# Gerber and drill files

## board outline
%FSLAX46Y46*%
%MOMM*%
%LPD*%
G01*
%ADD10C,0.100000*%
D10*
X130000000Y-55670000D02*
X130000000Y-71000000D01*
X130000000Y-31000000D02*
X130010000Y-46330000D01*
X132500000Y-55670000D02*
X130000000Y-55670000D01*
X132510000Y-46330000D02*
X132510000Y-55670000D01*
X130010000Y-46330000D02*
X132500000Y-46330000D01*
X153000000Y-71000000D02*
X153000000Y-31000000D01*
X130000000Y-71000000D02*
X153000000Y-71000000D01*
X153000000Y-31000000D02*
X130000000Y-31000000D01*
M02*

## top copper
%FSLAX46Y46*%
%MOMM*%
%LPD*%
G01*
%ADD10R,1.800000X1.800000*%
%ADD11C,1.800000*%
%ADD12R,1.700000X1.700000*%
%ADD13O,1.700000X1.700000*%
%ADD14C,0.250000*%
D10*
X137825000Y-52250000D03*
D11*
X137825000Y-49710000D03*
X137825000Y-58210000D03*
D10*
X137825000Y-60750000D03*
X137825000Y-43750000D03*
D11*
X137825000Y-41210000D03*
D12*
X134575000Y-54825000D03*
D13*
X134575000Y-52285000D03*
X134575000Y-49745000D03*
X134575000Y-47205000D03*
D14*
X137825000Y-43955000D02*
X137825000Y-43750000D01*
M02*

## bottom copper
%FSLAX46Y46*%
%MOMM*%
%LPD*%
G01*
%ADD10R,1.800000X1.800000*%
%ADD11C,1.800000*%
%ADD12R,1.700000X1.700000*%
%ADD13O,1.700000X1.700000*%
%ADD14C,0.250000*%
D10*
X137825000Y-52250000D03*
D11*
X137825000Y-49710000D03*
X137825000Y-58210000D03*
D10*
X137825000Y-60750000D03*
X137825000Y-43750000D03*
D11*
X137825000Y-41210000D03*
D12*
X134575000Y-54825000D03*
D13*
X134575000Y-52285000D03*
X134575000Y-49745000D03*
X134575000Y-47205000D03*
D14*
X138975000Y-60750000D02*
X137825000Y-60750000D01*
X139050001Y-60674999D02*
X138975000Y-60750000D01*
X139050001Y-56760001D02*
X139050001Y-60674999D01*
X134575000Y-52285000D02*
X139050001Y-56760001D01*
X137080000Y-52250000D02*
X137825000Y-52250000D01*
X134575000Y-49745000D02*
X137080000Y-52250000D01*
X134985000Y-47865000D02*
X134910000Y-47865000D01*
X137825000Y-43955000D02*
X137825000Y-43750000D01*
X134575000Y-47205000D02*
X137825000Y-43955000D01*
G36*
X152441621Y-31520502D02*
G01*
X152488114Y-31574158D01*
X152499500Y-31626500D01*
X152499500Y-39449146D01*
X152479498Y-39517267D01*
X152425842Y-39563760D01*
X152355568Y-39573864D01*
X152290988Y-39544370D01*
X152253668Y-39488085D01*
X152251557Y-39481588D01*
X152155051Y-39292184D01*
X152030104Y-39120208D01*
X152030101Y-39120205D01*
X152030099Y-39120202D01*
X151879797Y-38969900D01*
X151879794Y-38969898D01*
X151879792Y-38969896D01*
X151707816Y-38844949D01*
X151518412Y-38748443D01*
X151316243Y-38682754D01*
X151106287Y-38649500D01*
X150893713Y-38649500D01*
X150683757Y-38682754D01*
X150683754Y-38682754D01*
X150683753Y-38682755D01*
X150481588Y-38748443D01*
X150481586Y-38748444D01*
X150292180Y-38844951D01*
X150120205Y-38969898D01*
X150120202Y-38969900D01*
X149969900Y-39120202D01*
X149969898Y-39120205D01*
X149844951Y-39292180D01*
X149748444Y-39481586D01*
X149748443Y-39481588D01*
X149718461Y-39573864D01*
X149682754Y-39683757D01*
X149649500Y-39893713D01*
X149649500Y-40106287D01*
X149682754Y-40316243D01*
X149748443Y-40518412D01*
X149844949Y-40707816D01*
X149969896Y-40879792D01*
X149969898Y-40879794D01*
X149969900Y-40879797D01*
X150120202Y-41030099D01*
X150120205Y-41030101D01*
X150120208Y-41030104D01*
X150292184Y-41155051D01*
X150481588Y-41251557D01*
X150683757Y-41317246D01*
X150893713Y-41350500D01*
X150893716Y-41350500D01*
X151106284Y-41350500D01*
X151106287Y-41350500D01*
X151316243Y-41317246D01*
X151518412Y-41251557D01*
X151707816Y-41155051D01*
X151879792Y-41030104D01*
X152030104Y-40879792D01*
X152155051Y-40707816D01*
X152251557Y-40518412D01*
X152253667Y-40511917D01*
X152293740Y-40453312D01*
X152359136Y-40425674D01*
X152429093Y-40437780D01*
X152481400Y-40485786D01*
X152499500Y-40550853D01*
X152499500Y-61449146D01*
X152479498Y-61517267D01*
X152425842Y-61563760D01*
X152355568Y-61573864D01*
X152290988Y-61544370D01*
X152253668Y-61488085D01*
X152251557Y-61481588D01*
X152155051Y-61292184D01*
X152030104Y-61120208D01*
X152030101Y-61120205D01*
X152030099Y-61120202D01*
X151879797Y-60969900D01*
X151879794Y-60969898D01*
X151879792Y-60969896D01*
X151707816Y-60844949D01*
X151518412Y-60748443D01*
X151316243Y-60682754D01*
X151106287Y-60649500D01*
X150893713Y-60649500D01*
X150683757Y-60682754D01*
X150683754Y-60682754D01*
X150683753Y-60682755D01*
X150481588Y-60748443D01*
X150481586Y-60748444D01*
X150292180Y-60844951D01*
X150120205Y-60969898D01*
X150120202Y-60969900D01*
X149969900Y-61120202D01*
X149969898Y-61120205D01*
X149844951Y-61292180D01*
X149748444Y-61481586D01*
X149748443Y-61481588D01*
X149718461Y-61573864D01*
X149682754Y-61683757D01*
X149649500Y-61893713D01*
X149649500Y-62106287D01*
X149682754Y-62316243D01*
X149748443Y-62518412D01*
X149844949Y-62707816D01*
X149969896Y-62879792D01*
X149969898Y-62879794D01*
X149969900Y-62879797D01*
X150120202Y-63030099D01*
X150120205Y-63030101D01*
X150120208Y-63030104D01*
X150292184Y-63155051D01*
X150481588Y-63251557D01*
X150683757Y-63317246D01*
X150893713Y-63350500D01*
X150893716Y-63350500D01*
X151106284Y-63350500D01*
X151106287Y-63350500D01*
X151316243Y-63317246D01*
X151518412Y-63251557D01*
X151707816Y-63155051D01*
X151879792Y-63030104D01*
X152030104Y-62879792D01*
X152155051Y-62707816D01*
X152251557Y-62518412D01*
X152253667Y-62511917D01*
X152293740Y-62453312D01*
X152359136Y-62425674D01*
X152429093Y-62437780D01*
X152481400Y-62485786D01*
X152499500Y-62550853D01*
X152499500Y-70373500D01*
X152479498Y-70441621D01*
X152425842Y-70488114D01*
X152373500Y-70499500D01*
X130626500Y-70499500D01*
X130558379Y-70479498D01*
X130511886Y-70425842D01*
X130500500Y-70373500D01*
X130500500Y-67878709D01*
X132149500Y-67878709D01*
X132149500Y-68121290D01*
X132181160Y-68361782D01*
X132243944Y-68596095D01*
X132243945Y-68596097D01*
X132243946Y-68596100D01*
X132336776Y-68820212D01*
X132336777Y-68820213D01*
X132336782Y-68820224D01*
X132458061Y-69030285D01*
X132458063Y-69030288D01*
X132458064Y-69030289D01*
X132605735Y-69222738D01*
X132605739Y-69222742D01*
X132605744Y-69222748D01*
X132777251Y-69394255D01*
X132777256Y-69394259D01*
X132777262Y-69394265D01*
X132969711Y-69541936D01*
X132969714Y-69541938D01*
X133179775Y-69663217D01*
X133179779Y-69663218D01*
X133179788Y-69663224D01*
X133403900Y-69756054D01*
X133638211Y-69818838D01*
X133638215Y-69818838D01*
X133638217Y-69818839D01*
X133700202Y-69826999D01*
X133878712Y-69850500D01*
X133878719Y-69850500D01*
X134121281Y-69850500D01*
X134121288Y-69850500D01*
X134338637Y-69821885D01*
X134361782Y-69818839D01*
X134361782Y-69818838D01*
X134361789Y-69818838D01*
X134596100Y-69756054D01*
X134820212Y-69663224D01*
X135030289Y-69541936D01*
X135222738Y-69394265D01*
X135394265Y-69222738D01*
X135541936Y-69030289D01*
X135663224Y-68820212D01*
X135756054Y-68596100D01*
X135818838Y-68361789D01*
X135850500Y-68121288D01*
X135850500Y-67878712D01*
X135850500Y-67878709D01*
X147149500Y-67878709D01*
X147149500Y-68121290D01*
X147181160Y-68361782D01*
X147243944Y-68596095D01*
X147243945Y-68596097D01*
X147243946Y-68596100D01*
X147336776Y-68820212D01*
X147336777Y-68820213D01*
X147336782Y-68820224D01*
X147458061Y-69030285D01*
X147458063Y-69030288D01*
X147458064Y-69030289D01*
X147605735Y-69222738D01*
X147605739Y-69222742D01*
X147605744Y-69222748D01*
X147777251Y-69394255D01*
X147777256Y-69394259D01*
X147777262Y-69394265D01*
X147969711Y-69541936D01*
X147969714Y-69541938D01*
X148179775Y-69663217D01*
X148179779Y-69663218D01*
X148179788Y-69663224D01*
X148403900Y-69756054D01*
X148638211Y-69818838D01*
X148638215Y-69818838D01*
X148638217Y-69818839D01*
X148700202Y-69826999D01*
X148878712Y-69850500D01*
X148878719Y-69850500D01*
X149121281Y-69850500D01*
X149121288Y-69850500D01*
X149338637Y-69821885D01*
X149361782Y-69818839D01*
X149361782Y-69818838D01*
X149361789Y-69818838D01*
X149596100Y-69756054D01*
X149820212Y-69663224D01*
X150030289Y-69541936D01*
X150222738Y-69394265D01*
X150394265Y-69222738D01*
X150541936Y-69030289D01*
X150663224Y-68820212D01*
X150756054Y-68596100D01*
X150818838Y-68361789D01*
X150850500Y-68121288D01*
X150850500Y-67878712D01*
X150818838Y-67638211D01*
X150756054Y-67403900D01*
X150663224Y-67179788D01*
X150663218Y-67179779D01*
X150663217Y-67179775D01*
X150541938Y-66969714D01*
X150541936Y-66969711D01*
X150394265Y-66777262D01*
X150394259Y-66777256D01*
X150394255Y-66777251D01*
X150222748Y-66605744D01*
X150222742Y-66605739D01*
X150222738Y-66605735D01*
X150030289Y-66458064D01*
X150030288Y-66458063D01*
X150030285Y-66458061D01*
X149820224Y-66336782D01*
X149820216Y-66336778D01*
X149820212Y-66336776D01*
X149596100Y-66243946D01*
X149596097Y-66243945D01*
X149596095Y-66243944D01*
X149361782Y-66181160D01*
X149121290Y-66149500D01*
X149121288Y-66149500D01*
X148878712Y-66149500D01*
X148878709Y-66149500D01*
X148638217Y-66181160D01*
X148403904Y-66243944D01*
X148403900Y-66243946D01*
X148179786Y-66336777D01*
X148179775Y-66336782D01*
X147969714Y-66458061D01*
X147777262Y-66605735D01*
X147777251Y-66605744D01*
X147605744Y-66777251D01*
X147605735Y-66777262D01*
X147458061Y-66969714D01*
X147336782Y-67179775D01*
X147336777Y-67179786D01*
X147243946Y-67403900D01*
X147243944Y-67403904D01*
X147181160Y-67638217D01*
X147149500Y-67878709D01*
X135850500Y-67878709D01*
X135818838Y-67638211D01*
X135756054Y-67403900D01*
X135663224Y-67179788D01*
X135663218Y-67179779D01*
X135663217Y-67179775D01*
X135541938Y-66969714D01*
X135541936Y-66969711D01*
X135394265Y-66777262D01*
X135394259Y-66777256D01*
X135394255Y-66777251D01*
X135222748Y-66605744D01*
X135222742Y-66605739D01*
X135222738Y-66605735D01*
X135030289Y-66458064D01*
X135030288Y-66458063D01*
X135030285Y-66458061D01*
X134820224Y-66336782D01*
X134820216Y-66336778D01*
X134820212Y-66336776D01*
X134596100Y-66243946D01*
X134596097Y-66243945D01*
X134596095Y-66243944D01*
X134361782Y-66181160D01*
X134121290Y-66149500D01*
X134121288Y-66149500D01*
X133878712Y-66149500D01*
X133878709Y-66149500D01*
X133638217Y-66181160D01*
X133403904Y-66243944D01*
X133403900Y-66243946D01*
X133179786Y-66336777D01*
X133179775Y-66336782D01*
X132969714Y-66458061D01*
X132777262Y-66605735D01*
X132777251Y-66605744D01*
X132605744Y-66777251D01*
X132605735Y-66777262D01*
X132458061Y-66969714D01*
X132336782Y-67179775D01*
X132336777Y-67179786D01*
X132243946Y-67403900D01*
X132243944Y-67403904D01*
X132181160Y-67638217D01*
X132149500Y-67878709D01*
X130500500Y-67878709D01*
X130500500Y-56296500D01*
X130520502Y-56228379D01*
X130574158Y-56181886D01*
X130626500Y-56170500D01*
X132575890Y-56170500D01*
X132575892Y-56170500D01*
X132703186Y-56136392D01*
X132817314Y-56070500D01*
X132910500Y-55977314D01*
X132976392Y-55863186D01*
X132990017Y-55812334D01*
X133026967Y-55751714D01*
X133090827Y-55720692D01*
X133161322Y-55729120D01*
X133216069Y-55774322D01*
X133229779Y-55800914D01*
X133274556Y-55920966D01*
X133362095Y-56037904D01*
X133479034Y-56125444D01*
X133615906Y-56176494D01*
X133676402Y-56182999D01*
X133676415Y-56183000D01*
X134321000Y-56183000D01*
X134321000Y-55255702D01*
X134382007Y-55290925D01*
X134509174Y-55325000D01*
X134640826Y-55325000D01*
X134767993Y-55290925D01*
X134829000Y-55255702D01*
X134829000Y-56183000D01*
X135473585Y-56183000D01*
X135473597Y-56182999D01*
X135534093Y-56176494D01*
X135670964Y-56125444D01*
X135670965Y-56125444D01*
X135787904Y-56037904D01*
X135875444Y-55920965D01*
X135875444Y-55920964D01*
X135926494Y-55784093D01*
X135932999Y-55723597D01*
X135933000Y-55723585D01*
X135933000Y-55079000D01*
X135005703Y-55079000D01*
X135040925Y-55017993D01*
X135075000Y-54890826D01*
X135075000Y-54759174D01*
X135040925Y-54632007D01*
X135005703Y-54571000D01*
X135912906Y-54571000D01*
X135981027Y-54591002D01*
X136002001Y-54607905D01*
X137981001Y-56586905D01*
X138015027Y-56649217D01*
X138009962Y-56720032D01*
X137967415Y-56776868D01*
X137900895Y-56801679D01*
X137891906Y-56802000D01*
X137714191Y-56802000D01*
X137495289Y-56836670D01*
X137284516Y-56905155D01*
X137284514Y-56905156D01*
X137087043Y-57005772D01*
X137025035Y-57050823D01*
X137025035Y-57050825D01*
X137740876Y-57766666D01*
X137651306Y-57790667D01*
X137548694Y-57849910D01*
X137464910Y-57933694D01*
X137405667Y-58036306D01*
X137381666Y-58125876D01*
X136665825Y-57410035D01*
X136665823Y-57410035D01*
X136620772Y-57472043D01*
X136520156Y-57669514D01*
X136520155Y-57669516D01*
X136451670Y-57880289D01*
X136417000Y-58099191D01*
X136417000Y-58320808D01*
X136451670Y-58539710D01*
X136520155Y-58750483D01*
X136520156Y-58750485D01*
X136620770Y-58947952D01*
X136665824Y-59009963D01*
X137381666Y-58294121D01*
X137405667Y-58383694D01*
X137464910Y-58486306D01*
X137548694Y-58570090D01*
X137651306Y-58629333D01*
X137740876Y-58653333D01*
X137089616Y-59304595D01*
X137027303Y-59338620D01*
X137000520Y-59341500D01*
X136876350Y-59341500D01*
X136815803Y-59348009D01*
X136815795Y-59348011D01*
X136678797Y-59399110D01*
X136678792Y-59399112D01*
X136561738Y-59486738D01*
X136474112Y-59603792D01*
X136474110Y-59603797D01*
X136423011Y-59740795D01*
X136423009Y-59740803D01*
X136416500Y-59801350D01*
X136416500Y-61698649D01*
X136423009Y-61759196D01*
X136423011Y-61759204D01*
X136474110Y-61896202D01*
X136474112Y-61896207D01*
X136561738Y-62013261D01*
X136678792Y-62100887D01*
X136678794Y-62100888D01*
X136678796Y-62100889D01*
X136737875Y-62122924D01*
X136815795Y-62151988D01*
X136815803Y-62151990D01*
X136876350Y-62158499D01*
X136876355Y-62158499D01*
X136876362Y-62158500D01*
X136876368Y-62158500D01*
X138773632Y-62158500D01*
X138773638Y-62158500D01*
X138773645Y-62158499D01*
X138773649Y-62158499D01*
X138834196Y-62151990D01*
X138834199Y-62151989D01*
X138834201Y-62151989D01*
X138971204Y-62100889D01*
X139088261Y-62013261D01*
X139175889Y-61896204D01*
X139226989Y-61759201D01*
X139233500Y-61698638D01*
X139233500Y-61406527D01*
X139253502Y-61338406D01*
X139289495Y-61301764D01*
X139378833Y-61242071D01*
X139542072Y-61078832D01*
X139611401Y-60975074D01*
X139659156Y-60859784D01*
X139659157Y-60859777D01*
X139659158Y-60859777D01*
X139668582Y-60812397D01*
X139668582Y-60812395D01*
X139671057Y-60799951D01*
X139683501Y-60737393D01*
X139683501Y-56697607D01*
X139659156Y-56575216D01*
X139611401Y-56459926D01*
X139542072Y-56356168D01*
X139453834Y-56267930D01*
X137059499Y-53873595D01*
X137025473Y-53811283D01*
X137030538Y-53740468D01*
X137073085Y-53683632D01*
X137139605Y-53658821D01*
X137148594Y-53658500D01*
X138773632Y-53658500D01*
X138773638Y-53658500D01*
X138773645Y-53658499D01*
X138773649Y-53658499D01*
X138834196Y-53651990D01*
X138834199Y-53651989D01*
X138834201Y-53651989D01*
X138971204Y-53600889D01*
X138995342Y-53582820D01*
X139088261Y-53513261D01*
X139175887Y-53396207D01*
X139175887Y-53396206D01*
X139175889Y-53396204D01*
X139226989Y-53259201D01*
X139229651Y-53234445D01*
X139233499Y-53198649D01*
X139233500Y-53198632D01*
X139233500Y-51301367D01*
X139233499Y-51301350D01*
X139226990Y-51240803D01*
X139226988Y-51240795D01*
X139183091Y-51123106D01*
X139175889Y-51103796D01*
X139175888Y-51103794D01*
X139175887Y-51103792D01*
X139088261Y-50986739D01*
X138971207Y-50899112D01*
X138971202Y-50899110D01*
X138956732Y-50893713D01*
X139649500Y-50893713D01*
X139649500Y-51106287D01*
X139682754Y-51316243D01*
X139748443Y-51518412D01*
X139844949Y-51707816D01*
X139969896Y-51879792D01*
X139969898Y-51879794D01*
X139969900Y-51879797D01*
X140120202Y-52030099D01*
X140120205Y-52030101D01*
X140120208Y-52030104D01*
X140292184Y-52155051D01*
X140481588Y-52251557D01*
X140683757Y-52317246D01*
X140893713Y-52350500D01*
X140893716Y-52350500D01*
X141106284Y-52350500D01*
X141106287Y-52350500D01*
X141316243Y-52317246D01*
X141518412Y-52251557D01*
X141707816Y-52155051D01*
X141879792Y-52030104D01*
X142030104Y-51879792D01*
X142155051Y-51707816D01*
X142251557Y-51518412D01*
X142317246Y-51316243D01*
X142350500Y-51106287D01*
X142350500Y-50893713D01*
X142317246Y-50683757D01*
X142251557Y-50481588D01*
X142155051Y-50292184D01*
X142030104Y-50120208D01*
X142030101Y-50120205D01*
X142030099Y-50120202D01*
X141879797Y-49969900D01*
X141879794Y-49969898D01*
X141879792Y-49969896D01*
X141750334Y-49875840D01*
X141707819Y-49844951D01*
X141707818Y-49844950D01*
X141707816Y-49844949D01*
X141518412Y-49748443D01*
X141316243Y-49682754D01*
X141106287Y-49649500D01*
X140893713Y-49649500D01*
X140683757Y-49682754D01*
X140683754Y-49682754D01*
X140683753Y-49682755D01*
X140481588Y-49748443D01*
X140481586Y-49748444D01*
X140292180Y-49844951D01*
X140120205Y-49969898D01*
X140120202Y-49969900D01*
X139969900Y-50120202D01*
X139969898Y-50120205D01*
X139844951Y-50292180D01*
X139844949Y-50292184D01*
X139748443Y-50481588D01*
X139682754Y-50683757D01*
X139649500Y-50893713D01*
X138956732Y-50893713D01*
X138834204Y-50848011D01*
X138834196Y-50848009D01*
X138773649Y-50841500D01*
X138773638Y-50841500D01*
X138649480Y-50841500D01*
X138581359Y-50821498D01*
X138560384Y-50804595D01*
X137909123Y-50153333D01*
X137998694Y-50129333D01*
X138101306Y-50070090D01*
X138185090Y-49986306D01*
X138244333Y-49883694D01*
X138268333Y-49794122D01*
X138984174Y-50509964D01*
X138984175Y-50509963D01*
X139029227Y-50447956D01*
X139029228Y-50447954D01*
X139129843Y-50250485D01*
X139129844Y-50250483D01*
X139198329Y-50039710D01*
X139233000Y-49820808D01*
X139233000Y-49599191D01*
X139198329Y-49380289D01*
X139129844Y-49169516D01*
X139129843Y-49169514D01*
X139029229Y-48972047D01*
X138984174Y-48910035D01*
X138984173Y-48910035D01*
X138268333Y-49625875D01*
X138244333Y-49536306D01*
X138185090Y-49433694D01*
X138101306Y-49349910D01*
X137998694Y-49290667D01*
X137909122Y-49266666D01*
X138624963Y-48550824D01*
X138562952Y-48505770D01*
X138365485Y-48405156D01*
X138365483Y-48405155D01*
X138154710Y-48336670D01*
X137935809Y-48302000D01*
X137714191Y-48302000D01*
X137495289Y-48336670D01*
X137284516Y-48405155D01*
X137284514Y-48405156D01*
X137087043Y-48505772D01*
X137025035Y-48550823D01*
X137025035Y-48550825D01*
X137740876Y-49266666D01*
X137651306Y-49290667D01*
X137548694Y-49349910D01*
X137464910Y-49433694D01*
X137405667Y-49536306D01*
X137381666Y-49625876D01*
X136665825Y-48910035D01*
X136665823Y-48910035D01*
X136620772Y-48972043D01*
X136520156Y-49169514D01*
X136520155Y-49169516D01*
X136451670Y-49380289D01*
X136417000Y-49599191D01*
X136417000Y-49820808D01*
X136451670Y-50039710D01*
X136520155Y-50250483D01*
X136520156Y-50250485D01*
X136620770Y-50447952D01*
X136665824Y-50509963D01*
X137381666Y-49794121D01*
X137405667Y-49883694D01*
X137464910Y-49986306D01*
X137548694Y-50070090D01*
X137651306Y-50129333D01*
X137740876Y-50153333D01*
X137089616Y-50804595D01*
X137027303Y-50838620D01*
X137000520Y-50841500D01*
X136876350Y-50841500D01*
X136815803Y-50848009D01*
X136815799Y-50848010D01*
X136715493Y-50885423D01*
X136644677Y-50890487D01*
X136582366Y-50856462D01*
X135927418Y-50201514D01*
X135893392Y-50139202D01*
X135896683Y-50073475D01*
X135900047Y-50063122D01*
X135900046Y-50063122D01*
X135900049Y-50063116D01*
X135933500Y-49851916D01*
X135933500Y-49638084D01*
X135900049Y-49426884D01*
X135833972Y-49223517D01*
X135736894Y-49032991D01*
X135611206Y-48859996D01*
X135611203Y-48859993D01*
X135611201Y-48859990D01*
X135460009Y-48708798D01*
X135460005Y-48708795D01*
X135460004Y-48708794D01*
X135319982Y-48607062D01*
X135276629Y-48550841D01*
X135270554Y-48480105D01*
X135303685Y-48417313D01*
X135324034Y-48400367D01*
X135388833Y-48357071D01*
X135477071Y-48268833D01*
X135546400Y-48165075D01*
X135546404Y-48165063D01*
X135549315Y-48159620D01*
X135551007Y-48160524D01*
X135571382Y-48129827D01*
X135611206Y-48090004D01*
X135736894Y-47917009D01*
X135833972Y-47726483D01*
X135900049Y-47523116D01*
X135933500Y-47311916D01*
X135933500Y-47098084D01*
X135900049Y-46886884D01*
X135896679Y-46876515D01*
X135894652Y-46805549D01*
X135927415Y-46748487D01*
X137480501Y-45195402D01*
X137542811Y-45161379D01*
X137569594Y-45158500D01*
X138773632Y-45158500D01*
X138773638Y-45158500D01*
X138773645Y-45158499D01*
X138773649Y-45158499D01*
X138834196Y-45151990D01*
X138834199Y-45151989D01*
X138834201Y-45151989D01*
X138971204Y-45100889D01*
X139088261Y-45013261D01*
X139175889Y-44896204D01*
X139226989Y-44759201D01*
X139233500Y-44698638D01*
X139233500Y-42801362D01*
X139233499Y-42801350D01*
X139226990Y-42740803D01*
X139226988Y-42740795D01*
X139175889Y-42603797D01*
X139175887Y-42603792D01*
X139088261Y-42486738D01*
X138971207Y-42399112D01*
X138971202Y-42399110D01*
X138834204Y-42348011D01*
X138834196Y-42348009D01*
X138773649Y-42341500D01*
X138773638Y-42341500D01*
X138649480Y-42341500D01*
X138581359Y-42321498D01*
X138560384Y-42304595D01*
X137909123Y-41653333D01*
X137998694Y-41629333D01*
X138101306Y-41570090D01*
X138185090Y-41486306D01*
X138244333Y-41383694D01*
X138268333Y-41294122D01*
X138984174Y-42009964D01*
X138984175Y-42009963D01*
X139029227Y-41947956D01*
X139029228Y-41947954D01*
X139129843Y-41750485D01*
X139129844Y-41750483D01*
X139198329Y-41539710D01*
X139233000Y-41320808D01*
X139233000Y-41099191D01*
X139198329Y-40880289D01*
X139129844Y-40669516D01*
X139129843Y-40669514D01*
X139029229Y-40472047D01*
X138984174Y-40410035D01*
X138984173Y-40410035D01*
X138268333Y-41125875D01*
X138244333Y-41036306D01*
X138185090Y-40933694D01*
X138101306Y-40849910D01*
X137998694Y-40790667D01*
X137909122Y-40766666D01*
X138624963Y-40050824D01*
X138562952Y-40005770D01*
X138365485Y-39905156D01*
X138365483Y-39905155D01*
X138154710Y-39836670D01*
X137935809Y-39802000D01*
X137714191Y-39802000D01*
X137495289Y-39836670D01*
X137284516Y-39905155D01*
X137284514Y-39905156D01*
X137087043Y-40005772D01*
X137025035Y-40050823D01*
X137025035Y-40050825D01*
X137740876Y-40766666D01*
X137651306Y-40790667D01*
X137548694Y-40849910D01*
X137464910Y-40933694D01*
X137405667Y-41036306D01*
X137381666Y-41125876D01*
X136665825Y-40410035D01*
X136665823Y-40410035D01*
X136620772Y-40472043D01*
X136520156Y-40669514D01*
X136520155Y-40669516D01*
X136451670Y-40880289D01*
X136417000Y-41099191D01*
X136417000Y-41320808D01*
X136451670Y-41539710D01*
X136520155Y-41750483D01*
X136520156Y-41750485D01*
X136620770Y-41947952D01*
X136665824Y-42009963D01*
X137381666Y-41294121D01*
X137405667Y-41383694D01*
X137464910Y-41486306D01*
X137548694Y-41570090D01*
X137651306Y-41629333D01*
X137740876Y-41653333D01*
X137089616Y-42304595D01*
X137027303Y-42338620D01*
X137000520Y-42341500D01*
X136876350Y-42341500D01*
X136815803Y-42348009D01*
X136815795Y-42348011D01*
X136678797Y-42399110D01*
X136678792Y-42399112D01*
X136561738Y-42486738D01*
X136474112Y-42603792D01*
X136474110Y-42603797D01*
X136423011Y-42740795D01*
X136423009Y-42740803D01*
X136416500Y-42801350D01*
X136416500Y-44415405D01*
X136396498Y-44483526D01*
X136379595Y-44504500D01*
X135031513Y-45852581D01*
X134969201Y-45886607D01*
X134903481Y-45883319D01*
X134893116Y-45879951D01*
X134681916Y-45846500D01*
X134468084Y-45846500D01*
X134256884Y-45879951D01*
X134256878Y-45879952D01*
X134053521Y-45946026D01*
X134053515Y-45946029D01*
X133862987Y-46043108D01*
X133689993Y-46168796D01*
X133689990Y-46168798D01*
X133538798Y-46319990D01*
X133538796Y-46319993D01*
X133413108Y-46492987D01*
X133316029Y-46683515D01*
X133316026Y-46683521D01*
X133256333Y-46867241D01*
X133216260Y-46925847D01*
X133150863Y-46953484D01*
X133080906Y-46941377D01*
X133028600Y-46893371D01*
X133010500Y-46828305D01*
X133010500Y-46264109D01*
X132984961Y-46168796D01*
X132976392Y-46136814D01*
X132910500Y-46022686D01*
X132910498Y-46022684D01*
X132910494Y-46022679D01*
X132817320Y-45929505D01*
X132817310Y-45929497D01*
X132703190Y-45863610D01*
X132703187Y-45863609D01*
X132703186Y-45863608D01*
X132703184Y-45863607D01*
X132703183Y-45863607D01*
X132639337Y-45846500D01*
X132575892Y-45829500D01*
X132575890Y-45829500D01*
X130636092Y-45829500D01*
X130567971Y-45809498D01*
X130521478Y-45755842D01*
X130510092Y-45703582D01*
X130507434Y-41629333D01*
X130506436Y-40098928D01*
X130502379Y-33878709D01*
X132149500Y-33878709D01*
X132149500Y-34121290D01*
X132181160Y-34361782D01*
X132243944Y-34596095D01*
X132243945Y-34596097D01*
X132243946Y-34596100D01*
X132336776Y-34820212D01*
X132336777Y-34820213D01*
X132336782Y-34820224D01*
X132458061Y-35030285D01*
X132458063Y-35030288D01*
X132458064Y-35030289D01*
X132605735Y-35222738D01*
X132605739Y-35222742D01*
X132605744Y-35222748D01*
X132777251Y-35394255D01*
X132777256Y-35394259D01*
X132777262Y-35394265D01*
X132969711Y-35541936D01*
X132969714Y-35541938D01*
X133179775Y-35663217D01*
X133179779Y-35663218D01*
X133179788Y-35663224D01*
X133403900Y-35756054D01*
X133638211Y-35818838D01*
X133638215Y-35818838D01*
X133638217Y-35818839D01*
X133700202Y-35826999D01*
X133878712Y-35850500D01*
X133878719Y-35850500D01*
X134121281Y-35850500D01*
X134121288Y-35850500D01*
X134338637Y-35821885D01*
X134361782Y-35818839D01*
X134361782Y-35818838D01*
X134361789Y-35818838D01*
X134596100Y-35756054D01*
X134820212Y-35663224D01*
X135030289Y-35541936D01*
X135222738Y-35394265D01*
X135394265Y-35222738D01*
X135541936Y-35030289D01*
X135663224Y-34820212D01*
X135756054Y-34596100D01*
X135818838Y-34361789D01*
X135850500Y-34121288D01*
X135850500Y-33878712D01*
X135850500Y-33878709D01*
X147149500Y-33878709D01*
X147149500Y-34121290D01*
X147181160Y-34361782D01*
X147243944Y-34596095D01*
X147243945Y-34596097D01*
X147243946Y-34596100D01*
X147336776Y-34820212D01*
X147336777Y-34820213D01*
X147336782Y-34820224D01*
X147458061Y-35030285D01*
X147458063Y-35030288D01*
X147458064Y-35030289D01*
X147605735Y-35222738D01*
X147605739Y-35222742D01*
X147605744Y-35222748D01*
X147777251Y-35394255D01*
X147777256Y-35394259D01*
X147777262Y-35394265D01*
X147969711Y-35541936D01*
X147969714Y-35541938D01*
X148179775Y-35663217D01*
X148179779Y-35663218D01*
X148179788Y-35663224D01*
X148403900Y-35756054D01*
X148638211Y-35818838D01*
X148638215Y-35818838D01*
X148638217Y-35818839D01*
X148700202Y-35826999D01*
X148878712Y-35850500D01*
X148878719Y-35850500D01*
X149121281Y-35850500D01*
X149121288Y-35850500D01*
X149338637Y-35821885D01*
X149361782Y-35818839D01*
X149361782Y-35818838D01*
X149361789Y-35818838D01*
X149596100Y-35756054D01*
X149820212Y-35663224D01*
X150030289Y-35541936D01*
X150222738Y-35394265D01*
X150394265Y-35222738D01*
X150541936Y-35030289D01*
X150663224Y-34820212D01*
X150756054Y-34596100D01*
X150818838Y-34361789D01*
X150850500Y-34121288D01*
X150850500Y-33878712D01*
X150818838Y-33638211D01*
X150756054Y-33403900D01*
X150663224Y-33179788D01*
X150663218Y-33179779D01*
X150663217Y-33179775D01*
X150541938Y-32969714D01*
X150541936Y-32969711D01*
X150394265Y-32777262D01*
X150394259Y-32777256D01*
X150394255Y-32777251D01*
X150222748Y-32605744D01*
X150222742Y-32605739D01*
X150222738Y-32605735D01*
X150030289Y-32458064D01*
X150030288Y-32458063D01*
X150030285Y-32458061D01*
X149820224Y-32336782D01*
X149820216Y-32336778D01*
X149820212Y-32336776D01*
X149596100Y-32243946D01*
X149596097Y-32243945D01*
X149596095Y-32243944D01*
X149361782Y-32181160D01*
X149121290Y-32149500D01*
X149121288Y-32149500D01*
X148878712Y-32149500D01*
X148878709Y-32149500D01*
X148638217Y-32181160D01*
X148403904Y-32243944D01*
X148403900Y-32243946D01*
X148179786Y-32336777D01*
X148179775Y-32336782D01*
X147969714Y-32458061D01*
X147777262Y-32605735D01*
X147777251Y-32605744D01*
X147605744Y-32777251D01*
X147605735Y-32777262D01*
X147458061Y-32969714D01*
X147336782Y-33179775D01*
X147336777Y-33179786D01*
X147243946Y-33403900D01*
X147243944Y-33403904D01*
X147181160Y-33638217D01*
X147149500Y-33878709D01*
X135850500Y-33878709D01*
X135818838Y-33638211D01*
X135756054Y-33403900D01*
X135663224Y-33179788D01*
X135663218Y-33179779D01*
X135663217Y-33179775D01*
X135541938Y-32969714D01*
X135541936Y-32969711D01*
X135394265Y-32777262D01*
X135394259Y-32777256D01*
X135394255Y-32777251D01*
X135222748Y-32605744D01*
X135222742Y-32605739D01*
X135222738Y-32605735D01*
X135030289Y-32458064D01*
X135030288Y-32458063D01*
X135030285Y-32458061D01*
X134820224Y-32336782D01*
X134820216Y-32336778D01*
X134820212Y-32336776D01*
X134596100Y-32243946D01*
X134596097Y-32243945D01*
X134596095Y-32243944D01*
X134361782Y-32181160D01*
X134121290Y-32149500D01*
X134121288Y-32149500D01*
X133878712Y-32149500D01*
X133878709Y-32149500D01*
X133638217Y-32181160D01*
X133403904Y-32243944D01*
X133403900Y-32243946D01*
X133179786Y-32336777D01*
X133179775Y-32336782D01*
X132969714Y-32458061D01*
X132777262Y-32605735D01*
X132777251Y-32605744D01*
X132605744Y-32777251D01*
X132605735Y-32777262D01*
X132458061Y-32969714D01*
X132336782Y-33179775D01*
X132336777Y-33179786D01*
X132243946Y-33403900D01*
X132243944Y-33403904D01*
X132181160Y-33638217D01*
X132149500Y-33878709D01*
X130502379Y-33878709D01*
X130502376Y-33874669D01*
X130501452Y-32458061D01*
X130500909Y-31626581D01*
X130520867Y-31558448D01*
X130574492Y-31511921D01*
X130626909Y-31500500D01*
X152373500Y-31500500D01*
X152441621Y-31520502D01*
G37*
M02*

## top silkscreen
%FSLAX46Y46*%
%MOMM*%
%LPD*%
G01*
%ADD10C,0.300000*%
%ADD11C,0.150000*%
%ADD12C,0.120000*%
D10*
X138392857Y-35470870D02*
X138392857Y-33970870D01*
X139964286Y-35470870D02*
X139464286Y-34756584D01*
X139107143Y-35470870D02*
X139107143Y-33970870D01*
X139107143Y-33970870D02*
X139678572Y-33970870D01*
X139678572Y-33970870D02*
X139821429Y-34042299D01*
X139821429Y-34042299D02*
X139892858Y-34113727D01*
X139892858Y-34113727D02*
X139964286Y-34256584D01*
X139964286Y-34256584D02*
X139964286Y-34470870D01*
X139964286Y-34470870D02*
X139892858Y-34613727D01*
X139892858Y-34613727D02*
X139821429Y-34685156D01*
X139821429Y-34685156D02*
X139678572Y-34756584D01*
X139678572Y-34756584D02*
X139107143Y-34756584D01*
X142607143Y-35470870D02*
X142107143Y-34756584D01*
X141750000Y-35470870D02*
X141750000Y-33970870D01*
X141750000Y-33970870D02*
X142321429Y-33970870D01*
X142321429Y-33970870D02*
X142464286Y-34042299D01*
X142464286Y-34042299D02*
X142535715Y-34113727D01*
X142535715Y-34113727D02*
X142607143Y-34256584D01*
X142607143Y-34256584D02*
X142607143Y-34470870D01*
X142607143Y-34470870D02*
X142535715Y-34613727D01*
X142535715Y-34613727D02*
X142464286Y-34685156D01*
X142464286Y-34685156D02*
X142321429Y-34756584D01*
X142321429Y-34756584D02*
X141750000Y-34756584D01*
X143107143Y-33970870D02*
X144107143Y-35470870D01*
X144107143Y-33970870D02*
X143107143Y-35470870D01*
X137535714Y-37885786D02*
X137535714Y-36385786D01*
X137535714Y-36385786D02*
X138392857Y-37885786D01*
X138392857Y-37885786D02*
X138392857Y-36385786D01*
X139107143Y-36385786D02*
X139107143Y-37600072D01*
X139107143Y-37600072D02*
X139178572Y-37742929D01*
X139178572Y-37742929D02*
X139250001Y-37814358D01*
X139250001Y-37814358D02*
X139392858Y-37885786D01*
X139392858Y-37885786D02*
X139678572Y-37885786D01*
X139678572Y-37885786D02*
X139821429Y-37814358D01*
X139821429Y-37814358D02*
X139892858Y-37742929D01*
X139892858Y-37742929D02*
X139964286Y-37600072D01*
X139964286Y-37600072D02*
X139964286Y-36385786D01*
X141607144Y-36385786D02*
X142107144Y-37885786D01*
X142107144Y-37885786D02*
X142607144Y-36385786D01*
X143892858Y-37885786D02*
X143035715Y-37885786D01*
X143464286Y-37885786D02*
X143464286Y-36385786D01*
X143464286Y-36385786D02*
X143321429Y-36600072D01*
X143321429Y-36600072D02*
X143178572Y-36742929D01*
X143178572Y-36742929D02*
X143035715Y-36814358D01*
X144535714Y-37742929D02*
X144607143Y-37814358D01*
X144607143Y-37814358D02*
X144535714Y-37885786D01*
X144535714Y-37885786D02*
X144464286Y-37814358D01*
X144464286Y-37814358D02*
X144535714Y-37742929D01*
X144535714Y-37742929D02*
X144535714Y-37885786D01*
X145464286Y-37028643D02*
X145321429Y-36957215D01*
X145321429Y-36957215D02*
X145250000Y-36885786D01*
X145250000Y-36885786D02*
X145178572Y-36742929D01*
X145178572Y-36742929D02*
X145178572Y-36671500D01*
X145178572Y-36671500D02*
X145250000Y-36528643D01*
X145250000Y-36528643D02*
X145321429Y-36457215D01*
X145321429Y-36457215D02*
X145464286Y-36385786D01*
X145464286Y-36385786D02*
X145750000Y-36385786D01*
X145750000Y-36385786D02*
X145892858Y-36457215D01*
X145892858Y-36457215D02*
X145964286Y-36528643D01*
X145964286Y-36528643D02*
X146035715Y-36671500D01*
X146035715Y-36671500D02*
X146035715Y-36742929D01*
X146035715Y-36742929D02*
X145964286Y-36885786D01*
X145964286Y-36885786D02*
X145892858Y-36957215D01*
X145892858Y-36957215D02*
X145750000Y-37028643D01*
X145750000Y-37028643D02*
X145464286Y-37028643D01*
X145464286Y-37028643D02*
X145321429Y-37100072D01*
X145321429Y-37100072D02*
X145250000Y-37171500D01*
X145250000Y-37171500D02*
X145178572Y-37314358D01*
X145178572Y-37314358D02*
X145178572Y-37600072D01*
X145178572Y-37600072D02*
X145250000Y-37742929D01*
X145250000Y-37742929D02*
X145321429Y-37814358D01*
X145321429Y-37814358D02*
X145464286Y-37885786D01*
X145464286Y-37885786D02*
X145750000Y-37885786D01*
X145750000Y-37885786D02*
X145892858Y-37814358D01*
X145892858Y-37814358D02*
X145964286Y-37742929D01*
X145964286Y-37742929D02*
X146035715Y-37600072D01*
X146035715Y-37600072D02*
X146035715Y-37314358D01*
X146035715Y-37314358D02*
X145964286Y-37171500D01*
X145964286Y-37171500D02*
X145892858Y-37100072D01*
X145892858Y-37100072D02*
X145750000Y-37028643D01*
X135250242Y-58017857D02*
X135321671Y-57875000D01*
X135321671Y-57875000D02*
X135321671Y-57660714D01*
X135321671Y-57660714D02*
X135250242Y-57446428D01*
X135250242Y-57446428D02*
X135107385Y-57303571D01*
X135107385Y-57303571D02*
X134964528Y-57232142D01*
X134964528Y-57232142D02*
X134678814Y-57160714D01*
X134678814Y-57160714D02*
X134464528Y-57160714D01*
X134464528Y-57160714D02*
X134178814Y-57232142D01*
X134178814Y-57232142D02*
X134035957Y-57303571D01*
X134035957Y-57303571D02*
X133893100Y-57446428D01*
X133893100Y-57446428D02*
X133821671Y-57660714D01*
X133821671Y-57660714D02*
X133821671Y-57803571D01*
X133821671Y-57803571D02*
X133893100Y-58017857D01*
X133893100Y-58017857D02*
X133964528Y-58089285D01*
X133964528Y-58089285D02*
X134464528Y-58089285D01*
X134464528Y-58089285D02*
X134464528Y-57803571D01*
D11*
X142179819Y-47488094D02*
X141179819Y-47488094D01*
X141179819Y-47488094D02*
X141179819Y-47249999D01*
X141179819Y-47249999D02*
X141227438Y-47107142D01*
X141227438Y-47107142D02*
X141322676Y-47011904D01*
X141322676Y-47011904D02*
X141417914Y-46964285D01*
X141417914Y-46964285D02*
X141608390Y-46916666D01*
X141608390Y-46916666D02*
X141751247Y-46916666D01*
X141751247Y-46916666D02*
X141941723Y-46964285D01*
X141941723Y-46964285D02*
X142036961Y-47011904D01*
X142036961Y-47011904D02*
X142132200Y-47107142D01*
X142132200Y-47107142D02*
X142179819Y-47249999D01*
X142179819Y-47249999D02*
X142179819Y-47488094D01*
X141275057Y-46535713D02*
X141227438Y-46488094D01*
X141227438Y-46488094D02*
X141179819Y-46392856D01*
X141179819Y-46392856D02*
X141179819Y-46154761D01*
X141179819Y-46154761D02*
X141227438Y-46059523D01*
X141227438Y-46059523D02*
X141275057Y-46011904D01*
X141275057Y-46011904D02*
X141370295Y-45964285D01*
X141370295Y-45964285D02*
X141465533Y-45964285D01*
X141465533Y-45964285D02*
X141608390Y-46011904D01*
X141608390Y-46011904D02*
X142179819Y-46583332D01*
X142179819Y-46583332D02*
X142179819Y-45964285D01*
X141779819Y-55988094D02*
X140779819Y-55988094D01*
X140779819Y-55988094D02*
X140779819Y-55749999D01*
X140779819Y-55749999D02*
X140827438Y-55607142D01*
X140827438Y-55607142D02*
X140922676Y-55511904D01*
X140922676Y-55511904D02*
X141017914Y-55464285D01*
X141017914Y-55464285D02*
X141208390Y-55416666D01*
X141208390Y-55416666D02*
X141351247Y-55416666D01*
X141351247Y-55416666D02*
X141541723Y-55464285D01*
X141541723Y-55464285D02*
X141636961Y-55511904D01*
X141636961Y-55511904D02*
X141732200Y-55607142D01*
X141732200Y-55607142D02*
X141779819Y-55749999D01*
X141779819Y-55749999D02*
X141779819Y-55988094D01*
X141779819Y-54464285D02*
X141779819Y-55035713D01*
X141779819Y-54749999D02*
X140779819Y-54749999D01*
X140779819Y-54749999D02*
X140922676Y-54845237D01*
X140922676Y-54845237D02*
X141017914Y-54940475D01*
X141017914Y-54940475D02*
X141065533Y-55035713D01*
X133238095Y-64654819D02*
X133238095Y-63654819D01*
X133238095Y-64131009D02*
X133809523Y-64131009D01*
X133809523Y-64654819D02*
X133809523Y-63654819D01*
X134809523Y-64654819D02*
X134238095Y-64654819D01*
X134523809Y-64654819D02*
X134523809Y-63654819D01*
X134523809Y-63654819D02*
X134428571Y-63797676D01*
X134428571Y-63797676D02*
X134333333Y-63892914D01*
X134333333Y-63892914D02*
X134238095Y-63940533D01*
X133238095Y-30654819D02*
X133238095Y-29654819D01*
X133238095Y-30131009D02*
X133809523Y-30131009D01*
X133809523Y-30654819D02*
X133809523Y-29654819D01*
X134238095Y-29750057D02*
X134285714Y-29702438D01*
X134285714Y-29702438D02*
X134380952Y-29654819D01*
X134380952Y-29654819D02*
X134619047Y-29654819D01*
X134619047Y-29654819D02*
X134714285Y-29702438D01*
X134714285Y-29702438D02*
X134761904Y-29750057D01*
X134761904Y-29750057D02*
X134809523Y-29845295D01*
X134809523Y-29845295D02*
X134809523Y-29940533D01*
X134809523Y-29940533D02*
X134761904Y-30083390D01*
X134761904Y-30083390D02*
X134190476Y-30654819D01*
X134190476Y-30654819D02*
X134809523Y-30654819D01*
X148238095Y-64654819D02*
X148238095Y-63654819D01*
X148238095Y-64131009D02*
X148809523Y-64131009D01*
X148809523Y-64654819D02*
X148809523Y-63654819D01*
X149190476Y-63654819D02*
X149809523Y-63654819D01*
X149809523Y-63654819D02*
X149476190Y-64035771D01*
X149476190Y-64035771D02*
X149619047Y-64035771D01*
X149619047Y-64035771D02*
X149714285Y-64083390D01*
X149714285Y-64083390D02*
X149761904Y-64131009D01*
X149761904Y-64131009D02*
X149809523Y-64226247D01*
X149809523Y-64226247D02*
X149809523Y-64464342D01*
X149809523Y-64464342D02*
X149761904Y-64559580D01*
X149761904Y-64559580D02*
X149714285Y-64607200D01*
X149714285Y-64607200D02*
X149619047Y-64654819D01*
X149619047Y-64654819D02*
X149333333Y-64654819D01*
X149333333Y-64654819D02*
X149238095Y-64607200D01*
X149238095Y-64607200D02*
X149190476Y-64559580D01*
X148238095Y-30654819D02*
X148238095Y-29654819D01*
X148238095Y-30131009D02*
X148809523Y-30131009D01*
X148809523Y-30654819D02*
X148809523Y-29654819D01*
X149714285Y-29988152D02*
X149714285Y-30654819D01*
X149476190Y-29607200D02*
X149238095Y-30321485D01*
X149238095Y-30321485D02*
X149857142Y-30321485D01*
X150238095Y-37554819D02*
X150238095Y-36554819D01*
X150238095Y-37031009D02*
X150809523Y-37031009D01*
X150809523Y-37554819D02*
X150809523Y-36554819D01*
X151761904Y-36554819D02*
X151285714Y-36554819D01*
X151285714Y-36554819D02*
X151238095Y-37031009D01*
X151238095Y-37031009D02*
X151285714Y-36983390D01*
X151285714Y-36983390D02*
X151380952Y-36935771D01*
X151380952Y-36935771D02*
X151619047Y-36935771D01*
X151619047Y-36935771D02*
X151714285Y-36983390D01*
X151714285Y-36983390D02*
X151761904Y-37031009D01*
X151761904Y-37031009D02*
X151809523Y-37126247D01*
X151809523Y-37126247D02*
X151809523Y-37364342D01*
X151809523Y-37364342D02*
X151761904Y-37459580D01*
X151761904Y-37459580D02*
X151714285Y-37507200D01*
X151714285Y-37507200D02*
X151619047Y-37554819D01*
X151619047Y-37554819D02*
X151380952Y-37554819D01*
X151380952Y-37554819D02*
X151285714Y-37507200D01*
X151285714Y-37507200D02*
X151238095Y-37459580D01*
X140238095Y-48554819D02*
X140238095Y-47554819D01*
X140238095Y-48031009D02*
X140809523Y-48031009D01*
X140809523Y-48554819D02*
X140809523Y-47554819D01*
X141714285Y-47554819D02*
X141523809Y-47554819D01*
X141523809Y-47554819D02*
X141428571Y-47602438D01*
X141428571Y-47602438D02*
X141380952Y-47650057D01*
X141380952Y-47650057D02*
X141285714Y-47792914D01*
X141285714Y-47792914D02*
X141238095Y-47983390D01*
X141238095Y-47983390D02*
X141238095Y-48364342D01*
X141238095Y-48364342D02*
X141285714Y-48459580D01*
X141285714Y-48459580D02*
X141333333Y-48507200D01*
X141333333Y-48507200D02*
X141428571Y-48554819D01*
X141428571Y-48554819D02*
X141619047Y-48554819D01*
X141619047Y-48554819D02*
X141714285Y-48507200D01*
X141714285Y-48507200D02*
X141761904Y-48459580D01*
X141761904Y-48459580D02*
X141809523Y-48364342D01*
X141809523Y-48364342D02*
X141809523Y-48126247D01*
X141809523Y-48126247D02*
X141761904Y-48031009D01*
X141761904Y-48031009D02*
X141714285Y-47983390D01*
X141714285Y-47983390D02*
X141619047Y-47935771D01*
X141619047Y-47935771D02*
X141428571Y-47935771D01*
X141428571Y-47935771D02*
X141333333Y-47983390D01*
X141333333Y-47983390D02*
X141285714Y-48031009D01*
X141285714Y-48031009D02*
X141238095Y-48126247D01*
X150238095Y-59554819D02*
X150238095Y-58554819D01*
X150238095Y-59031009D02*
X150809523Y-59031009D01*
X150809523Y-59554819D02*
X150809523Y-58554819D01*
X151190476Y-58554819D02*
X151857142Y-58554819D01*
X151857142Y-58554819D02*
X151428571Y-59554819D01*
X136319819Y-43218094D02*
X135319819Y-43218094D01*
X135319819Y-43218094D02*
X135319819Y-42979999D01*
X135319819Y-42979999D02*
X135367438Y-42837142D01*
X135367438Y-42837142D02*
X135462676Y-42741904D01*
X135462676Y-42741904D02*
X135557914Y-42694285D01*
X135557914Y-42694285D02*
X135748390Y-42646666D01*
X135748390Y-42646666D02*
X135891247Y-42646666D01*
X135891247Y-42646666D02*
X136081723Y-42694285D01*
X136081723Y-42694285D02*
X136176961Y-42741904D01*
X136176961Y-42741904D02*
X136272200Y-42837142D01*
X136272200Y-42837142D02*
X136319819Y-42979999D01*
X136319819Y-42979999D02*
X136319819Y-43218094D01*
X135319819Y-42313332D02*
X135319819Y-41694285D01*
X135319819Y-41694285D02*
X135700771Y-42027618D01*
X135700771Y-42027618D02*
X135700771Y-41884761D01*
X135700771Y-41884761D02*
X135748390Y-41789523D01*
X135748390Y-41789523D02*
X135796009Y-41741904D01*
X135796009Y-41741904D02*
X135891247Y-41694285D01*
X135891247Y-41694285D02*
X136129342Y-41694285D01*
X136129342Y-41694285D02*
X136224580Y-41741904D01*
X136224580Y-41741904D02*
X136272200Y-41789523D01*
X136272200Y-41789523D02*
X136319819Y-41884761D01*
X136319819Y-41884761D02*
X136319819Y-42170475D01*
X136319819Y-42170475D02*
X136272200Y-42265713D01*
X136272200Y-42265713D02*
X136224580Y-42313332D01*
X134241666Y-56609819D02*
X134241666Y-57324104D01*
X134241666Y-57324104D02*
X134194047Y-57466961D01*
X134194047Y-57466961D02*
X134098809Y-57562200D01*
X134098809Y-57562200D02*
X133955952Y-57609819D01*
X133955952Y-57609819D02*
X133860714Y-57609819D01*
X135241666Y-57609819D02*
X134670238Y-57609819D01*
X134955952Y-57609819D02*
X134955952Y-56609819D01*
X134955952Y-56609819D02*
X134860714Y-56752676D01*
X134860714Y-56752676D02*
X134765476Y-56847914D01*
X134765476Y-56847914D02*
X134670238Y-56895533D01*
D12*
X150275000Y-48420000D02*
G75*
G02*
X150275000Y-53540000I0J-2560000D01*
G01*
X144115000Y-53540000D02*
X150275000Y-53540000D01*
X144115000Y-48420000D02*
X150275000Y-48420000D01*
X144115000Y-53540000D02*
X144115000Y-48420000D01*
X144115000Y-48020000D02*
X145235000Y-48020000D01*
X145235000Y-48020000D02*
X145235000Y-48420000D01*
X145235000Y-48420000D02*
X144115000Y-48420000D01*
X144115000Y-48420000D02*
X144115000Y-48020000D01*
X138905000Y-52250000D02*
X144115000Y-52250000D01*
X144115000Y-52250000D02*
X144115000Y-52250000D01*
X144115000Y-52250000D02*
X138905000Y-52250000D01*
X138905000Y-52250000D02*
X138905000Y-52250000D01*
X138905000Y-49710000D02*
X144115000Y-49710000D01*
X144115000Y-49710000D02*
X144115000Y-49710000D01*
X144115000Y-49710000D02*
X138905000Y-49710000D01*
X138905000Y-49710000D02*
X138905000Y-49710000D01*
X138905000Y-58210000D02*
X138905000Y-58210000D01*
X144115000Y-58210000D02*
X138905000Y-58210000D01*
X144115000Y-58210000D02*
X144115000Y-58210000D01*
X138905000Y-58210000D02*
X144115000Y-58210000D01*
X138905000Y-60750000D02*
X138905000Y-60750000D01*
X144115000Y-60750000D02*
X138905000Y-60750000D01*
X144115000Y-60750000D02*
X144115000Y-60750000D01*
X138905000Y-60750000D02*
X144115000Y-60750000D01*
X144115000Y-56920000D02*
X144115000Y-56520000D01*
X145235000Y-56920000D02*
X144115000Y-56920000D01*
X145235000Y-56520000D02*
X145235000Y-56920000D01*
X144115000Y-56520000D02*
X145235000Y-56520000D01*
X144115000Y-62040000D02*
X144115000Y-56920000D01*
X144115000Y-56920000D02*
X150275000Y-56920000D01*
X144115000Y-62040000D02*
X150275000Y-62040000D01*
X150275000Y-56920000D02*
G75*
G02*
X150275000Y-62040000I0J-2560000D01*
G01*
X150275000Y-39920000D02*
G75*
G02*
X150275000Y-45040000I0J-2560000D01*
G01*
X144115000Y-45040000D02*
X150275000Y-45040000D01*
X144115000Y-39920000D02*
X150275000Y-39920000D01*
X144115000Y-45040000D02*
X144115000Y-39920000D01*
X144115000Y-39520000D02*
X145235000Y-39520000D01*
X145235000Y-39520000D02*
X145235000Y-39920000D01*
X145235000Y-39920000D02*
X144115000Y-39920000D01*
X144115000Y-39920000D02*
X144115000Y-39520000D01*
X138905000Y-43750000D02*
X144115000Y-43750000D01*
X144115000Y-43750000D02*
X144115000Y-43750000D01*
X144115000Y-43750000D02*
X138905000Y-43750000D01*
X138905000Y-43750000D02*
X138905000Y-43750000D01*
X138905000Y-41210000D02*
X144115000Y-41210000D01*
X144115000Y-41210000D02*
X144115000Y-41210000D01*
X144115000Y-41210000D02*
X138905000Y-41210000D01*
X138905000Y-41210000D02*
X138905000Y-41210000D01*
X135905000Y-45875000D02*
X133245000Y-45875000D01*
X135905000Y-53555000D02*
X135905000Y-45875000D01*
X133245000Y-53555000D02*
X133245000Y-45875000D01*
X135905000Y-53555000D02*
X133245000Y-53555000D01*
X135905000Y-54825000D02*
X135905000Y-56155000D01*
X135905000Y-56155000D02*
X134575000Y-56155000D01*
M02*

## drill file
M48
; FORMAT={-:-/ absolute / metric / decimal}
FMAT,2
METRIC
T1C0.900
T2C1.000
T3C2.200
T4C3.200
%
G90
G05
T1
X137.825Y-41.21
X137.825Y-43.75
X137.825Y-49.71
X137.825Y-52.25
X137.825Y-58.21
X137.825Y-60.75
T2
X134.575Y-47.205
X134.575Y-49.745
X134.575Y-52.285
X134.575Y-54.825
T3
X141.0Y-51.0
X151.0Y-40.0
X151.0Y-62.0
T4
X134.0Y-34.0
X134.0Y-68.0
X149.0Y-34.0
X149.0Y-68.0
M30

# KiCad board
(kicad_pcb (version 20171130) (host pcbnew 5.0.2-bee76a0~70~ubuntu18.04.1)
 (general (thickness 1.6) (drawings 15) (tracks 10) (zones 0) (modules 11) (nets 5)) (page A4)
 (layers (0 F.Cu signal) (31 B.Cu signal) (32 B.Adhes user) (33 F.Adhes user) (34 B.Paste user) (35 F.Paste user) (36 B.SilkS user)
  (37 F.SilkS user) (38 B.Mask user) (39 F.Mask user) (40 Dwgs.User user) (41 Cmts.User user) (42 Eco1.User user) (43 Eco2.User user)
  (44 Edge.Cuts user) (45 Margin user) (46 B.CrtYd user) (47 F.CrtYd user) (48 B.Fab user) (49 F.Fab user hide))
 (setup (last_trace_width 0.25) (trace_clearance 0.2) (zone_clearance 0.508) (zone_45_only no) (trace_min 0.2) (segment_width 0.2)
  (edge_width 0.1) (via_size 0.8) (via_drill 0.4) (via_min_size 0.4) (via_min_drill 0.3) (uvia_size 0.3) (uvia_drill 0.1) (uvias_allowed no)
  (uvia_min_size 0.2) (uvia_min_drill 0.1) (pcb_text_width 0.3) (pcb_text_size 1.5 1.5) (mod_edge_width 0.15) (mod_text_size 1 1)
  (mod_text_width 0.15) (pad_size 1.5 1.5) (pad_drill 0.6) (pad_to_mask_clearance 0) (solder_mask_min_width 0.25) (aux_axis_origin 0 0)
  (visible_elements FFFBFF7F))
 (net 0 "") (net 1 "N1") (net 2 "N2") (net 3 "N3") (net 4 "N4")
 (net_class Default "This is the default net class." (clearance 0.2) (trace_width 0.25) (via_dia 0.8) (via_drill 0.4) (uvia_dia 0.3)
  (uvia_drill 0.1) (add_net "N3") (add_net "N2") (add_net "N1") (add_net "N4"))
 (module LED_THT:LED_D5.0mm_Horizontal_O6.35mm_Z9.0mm (layer F.Cu) (at 137.825 52.25 90)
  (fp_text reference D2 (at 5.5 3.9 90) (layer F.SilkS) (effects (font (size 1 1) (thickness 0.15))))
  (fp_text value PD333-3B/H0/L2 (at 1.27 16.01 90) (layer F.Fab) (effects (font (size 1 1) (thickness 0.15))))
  (fp_arc (start 1.27 12.45) (end -1.29 12.45) (angle -180) (layer F.SilkS) (width 0.12))
  (fp_line (start -1.29 6.29) (end -1.29 12.45) (layer F.SilkS) (width 0.12))
  (fp_line (start 3.83 6.29) (end 3.83 12.45) (layer F.SilkS) (width 0.12))
  (fp_line (start -1.29 6.29) (end 3.83 6.29) (layer F.SilkS) (width 0.12))
  (fp_line (start 4.23 6.29) (end 4.23 7.41) (layer F.SilkS) (width 0.12))
  (fp_line (start 4.23 7.41) (end 3.83 7.41) (layer F.SilkS) (width 0.12))
  (fp_line (start 3.83 7.41) (end 3.83 6.29) (layer F.SilkS) (width 0.12))
  (fp_line (start 3.83 6.29) (end 4.23 6.29) (layer F.SilkS) (width 0.12))
  (fp_line (start 0 1.08) (end 0 6.29) (layer F.SilkS) (width 0.12))
  (fp_line (start 0 6.29) (end 0 6.29) (layer F.SilkS) (width 0.12))
  (fp_line (start 0 6.29) (end 0 1.08) (layer F.SilkS) (width 0.12))
  (fp_line (start 0 1.08) (end 0 1.08) (layer F.SilkS) (width 0.12))
  (fp_line (start 2.54 1.08) (end 2.54 6.29) (layer F.SilkS) (width 0.12))
  (fp_line (start 2.54 6.29) (end 2.54 6.29) (layer F.SilkS) (width 0.12))
  (fp_line (start 2.54 6.29) (end 2.54 1.08) (layer F.SilkS) (width 0.12))
  (fp_line (start 2.54 1.08) (end 2.54 1.08) (layer F.SilkS) (width 0.12))
  (pad 1 thru_hole rect (at 0 0 90) (size 1.8 1.8) (drill 0.9) (layers *.Cu *.Mask) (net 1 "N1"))
  (pad 2 thru_hole circle (at 2.54 0 90) (size 1.8 1.8) (drill 0.9) (layers *.Cu *.Mask) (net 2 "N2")))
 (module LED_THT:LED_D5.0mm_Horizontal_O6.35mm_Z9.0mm (layer F.Cu) (at 137.825 60.75 90)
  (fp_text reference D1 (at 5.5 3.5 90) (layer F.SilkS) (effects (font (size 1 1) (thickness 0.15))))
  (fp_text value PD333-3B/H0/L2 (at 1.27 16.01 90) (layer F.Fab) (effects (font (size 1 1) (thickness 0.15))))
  (fp_line (start 2.54 1.08) (end 2.54 1.08) (layer F.SilkS) (width 0.12))
  (fp_line (start 2.54 6.29) (end 2.54 1.08) (layer F.SilkS) (width 0.12))
  (fp_line (start 2.54 6.29) (end 2.54 6.29) (layer F.SilkS) (width 0.12))
  (fp_line (start 2.54 1.08) (end 2.54 6.29) (layer F.SilkS) (width 0.12))
  (fp_line (start 0 1.08) (end 0 1.08) (layer F.SilkS) (width 0.12))
  (fp_line (start 0 6.29) (end 0 1.08) (layer F.SilkS) (width 0.12))
  (fp_line (start 0 6.29) (end 0 6.29) (layer F.SilkS) (width 0.12))
  (fp_line (start 0 1.08) (end 0 6.29) (layer F.SilkS) (width 0.12))
  (fp_line (start 3.83 6.29) (end 4.23 6.29) (layer F.SilkS) (width 0.12))
  (fp_line (start 3.83 7.41) (end 3.83 6.29) (layer F.SilkS) (width 0.12))
  (fp_line (start 4.23 7.41) (end 3.83 7.41) (layer F.SilkS) (width 0.12))
  (fp_line (start 4.23 6.29) (end 4.23 7.41) (layer F.SilkS) (width 0.12))
  (fp_line (start -1.29 6.29) (end 3.83 6.29) (layer F.SilkS) (width 0.12))
  (fp_line (start 3.83 6.29) (end 3.83 12.45) (layer F.SilkS) (width 0.12))
  (fp_line (start -1.29 6.29) (end -1.29 12.45) (layer F.SilkS) (width 0.12))
  (fp_arc (start 1.27 12.45) (end -1.29 12.45) (angle -180) (layer F.SilkS) (width 0.12))
  (pad 2 thru_hole circle (at 2.54 0 90) (size 1.8 1.8) (drill 0.9) (layers *.Cu *.Mask) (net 2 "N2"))
  (pad 1 thru_hole rect (at 0 0 90) (size 1.8 1.8) (drill 0.9) (layers *.Cu *.Mask) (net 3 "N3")))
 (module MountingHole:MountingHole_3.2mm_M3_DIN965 (layer F.Cu) (at 134 68)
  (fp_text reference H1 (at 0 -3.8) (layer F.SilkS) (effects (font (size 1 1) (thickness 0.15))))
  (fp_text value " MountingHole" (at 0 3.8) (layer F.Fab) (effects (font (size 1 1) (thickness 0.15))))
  (pad 1 np_thru_hole circle (at 0 0) (size 3.2 3.2) (drill 3.2) (layers *.Cu *.Mask)))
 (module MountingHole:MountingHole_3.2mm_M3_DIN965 (layer F.Cu) (at 134 34)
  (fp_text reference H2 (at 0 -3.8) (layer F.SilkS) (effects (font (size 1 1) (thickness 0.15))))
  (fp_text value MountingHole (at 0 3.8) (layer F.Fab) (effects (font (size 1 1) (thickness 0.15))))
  (pad 1 np_thru_hole circle (at 0 0) (size 3.2 3.2) (drill 3.2) (layers *.Cu *.Mask)))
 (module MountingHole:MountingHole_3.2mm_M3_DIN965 (layer F.Cu) (at 149 68)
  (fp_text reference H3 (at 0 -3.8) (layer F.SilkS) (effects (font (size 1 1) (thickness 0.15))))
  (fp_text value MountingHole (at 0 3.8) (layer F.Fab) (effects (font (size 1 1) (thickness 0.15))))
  (pad 1 np_thru_hole circle (at 0 0) (size 3.2 3.2) (drill 3.2) (layers *.Cu *.Mask)))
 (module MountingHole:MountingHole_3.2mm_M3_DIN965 (layer F.Cu) (at 149 34)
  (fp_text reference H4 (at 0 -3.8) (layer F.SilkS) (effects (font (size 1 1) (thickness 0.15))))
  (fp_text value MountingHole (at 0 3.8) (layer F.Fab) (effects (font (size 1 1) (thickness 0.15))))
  (pad 1 np_thru_hole circle (at 0 0) (size 3.2 3.2) (drill 3.2) (layers *.Cu *.Mask)))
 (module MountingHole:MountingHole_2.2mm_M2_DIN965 (layer F.Cu) (at 151 40)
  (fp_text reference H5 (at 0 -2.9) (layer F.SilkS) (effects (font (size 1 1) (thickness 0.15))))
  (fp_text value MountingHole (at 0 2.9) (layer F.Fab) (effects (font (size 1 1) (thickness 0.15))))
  (pad 1 np_thru_hole circle (at 0 0) (size 2.2 2.2) (drill 2.2) (layers *.Cu *.Mask)))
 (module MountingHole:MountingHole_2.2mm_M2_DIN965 (layer F.Cu) (at 141 51)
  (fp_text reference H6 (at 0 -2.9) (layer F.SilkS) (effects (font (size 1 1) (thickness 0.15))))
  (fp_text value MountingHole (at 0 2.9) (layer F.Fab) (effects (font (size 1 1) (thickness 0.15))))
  (pad 1 np_thru_hole circle (at 0 0) (size 2.2 2.2) (drill 2.2) (layers *.Cu *.Mask)))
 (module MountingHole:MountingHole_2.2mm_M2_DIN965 (layer F.Cu) (at 151 62)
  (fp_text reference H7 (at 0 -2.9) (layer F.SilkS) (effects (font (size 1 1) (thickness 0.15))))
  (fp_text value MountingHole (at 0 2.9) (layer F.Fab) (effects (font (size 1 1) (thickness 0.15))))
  (pad 1 np_thru_hole circle (at 0 0) (size 2.2 2.2) (drill 2.2) (layers *.Cu *.Mask)))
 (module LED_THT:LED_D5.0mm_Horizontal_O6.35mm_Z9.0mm (layer F.Cu) (at 137.825 43.75 90)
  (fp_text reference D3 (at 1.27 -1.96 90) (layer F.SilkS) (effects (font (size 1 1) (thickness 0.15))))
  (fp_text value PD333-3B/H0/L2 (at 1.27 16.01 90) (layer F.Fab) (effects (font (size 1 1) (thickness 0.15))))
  (fp_arc (start 1.27 12.45) (end -1.29 12.45) (angle -180) (layer F.SilkS) (width 0.12))
  (fp_line (start -1.29 6.29) (end -1.29 12.45) (layer F.SilkS) (width 0.12))
  (fp_line (start 3.83 6.29) (end 3.83 12.45) (layer F.SilkS) (width 0.12))
  (fp_line (start -1.29 6.29) (end 3.83 6.29) (layer F.SilkS) (width 0.12))
  (fp_line (start 4.23 6.29) (end 4.23 7.41) (layer F.SilkS) (width 0.12))
  (fp_line (start 4.23 7.41) (end 3.83 7.41) (layer F.SilkS) (width 0.12))
  (fp_line (start 3.83 7.41) (end 3.83 6.29) (layer F.SilkS) (width 0.12))
  (fp_line (start 3.83 6.29) (end 4.23 6.29) (layer F.SilkS) (width 0.12))
  (fp_line (start 0 1.08) (end 0 6.29) (layer F.SilkS) (width 0.12))
  (fp_line (start 0 6.29) (end 0 6.29) (layer F.SilkS) (width 0.12))
  (fp_line (start 0 6.29) (end 0 1.08) (layer F.SilkS) (width 0.12))
  (fp_line (start 0 1.08) (end 0 1.08) (layer F.SilkS) (width 0.12))
  (fp_line (start 2.54 1.08) (end 2.54 6.29) (layer F.SilkS) (width 0.12))
  (fp_line (start 2.54 6.29) (end 2.54 6.29) (layer F.SilkS) (width 0.12))
  (fp_line (start 2.54 6.29) (end 2.54 1.08) (layer F.SilkS) (width 0.12))
  (fp_line (start 2.54 1.08) (end 2.54 1.08) (layer F.SilkS) (width 0.12))
  (pad 1 thru_hole rect (at 0 0 90) (size 1.8 1.8) (drill 0.9) (layers *.Cu *.Mask) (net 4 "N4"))
  (pad 2 thru_hole circle (at 2.54 0 90) (size 1.8 1.8) (drill 0.9) (layers *.Cu *.Mask) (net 2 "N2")))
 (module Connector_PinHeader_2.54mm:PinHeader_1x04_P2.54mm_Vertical (layer F.Cu) (at 134.575 54.825 180)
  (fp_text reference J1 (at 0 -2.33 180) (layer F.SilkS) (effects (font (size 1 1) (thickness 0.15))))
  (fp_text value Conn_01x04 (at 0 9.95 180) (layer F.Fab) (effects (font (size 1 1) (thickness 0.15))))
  (fp_line (start -1.33 8.95) (end 1.33 8.95) (layer F.SilkS) (width 0.12))
  (fp_line (start -1.33 1.27) (end -1.33 8.95) (layer F.SilkS) (width 0.12))
  (fp_line (start 1.33 1.27) (end 1.33 8.95) (layer F.SilkS) (width 0.12))
  (fp_line (start -1.33 1.27) (end 1.33 1.27) (layer F.SilkS) (width 0.12))
  (fp_line (start -1.33 0) (end -1.33 -1.33) (layer F.SilkS) (width 0.12))
  (fp_line (start -1.33 -1.33) (end 0 -1.33) (layer F.SilkS) (width 0.12))
  (pad 1 thru_hole rect (at 0 0 180) (size 1.7 1.7) (drill 1) (layers *.Cu *.Mask) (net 2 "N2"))
  (pad 2 thru_hole oval (at 0 2.54 180) (size 1.7 1.7) (drill 1) (layers *.Cu *.Mask) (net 3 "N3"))
  (pad 3 thru_hole oval (at 0 5.08 180) (size 1.7 1.7) (drill 1) (layers *.Cu *.Mask) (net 1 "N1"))
  (pad 4 thru_hole oval (at 0 7.62 180) (size 1.7 1.7) (drill 1) (layers *.Cu *.Mask) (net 4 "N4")))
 (gr_line (start 130 55.67) (end 130 71) (layer Edge.Cuts) (width 0.1))
 (gr_line (start 130 31) (end 130.01 46.33) (layer Edge.Cuts) (width 0.1))
 (gr_line (start 132.5 55.67) (end 130 55.67) (layer Edge.Cuts) (width 0.1))
 (gr_line (start 132.51 46.33) (end 132.51 55.67) (layer Edge.Cuts) (width 0.1))
 (gr_line (start 130.01 46.33) (end 132.5 46.33) (layer Edge.Cuts) (width 0.1))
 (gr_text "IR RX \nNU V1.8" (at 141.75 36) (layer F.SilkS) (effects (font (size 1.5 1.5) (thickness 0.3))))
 (gr_line (start 153 71) (end 153 31) (layer Edge.Cuts) (width 0.1))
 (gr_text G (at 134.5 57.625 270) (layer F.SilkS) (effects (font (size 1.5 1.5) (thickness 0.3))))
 (gr_line (start 130 71) (end 153 71) (layer Edge.Cuts) (width 0.1))
 (gr_line (start 153 31) (end 130 31) (layer Edge.Cuts) (width 0.1))
 (segment (start 138.975 60.75) (end 137.825 60.75) (width 0.25) (layer B.Cu) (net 3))
 (segment (start 139.050001 60.674999) (end 138.975 60.75) (width 0.25) (layer B.Cu) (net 3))
 (segment (start 139.050001 56.760001) (end 139.050001 60.674999) (width 0.25) (layer B.Cu) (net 3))
 (segment (start 134.575 52.285) (end 139.050001 56.760001) (width 0.25) (layer B.Cu) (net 3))
 (segment (start 137.08 52.25) (end 137.825 52.25) (width 0.25) (layer B.Cu) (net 1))
 (segment (start 134.575 49.745) (end 137.08 52.25) (width 0.25) (layer B.Cu) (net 1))
 (segment (start 134.985 47.865) (end 134.91 47.865) (width 0.25) (layer B.Cu) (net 4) (status 30))
 (segment (start 137.825 43.955) (end 137.825 43.75) (width 0.25) (layer F.Cu) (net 4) (status 30))
 (segment (start 137.825 43.955) (end 137.825 43.75) (width 0.25) (layer B.Cu) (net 4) (status 30))
 (segment (start 134.575 47.205) (end 137.825 43.955) (width 0.25) (layer B.Cu) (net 4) (status 30))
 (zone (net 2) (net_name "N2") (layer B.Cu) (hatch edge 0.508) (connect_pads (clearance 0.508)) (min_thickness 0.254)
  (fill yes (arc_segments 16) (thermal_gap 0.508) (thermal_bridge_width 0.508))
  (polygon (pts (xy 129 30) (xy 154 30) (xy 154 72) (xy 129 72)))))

